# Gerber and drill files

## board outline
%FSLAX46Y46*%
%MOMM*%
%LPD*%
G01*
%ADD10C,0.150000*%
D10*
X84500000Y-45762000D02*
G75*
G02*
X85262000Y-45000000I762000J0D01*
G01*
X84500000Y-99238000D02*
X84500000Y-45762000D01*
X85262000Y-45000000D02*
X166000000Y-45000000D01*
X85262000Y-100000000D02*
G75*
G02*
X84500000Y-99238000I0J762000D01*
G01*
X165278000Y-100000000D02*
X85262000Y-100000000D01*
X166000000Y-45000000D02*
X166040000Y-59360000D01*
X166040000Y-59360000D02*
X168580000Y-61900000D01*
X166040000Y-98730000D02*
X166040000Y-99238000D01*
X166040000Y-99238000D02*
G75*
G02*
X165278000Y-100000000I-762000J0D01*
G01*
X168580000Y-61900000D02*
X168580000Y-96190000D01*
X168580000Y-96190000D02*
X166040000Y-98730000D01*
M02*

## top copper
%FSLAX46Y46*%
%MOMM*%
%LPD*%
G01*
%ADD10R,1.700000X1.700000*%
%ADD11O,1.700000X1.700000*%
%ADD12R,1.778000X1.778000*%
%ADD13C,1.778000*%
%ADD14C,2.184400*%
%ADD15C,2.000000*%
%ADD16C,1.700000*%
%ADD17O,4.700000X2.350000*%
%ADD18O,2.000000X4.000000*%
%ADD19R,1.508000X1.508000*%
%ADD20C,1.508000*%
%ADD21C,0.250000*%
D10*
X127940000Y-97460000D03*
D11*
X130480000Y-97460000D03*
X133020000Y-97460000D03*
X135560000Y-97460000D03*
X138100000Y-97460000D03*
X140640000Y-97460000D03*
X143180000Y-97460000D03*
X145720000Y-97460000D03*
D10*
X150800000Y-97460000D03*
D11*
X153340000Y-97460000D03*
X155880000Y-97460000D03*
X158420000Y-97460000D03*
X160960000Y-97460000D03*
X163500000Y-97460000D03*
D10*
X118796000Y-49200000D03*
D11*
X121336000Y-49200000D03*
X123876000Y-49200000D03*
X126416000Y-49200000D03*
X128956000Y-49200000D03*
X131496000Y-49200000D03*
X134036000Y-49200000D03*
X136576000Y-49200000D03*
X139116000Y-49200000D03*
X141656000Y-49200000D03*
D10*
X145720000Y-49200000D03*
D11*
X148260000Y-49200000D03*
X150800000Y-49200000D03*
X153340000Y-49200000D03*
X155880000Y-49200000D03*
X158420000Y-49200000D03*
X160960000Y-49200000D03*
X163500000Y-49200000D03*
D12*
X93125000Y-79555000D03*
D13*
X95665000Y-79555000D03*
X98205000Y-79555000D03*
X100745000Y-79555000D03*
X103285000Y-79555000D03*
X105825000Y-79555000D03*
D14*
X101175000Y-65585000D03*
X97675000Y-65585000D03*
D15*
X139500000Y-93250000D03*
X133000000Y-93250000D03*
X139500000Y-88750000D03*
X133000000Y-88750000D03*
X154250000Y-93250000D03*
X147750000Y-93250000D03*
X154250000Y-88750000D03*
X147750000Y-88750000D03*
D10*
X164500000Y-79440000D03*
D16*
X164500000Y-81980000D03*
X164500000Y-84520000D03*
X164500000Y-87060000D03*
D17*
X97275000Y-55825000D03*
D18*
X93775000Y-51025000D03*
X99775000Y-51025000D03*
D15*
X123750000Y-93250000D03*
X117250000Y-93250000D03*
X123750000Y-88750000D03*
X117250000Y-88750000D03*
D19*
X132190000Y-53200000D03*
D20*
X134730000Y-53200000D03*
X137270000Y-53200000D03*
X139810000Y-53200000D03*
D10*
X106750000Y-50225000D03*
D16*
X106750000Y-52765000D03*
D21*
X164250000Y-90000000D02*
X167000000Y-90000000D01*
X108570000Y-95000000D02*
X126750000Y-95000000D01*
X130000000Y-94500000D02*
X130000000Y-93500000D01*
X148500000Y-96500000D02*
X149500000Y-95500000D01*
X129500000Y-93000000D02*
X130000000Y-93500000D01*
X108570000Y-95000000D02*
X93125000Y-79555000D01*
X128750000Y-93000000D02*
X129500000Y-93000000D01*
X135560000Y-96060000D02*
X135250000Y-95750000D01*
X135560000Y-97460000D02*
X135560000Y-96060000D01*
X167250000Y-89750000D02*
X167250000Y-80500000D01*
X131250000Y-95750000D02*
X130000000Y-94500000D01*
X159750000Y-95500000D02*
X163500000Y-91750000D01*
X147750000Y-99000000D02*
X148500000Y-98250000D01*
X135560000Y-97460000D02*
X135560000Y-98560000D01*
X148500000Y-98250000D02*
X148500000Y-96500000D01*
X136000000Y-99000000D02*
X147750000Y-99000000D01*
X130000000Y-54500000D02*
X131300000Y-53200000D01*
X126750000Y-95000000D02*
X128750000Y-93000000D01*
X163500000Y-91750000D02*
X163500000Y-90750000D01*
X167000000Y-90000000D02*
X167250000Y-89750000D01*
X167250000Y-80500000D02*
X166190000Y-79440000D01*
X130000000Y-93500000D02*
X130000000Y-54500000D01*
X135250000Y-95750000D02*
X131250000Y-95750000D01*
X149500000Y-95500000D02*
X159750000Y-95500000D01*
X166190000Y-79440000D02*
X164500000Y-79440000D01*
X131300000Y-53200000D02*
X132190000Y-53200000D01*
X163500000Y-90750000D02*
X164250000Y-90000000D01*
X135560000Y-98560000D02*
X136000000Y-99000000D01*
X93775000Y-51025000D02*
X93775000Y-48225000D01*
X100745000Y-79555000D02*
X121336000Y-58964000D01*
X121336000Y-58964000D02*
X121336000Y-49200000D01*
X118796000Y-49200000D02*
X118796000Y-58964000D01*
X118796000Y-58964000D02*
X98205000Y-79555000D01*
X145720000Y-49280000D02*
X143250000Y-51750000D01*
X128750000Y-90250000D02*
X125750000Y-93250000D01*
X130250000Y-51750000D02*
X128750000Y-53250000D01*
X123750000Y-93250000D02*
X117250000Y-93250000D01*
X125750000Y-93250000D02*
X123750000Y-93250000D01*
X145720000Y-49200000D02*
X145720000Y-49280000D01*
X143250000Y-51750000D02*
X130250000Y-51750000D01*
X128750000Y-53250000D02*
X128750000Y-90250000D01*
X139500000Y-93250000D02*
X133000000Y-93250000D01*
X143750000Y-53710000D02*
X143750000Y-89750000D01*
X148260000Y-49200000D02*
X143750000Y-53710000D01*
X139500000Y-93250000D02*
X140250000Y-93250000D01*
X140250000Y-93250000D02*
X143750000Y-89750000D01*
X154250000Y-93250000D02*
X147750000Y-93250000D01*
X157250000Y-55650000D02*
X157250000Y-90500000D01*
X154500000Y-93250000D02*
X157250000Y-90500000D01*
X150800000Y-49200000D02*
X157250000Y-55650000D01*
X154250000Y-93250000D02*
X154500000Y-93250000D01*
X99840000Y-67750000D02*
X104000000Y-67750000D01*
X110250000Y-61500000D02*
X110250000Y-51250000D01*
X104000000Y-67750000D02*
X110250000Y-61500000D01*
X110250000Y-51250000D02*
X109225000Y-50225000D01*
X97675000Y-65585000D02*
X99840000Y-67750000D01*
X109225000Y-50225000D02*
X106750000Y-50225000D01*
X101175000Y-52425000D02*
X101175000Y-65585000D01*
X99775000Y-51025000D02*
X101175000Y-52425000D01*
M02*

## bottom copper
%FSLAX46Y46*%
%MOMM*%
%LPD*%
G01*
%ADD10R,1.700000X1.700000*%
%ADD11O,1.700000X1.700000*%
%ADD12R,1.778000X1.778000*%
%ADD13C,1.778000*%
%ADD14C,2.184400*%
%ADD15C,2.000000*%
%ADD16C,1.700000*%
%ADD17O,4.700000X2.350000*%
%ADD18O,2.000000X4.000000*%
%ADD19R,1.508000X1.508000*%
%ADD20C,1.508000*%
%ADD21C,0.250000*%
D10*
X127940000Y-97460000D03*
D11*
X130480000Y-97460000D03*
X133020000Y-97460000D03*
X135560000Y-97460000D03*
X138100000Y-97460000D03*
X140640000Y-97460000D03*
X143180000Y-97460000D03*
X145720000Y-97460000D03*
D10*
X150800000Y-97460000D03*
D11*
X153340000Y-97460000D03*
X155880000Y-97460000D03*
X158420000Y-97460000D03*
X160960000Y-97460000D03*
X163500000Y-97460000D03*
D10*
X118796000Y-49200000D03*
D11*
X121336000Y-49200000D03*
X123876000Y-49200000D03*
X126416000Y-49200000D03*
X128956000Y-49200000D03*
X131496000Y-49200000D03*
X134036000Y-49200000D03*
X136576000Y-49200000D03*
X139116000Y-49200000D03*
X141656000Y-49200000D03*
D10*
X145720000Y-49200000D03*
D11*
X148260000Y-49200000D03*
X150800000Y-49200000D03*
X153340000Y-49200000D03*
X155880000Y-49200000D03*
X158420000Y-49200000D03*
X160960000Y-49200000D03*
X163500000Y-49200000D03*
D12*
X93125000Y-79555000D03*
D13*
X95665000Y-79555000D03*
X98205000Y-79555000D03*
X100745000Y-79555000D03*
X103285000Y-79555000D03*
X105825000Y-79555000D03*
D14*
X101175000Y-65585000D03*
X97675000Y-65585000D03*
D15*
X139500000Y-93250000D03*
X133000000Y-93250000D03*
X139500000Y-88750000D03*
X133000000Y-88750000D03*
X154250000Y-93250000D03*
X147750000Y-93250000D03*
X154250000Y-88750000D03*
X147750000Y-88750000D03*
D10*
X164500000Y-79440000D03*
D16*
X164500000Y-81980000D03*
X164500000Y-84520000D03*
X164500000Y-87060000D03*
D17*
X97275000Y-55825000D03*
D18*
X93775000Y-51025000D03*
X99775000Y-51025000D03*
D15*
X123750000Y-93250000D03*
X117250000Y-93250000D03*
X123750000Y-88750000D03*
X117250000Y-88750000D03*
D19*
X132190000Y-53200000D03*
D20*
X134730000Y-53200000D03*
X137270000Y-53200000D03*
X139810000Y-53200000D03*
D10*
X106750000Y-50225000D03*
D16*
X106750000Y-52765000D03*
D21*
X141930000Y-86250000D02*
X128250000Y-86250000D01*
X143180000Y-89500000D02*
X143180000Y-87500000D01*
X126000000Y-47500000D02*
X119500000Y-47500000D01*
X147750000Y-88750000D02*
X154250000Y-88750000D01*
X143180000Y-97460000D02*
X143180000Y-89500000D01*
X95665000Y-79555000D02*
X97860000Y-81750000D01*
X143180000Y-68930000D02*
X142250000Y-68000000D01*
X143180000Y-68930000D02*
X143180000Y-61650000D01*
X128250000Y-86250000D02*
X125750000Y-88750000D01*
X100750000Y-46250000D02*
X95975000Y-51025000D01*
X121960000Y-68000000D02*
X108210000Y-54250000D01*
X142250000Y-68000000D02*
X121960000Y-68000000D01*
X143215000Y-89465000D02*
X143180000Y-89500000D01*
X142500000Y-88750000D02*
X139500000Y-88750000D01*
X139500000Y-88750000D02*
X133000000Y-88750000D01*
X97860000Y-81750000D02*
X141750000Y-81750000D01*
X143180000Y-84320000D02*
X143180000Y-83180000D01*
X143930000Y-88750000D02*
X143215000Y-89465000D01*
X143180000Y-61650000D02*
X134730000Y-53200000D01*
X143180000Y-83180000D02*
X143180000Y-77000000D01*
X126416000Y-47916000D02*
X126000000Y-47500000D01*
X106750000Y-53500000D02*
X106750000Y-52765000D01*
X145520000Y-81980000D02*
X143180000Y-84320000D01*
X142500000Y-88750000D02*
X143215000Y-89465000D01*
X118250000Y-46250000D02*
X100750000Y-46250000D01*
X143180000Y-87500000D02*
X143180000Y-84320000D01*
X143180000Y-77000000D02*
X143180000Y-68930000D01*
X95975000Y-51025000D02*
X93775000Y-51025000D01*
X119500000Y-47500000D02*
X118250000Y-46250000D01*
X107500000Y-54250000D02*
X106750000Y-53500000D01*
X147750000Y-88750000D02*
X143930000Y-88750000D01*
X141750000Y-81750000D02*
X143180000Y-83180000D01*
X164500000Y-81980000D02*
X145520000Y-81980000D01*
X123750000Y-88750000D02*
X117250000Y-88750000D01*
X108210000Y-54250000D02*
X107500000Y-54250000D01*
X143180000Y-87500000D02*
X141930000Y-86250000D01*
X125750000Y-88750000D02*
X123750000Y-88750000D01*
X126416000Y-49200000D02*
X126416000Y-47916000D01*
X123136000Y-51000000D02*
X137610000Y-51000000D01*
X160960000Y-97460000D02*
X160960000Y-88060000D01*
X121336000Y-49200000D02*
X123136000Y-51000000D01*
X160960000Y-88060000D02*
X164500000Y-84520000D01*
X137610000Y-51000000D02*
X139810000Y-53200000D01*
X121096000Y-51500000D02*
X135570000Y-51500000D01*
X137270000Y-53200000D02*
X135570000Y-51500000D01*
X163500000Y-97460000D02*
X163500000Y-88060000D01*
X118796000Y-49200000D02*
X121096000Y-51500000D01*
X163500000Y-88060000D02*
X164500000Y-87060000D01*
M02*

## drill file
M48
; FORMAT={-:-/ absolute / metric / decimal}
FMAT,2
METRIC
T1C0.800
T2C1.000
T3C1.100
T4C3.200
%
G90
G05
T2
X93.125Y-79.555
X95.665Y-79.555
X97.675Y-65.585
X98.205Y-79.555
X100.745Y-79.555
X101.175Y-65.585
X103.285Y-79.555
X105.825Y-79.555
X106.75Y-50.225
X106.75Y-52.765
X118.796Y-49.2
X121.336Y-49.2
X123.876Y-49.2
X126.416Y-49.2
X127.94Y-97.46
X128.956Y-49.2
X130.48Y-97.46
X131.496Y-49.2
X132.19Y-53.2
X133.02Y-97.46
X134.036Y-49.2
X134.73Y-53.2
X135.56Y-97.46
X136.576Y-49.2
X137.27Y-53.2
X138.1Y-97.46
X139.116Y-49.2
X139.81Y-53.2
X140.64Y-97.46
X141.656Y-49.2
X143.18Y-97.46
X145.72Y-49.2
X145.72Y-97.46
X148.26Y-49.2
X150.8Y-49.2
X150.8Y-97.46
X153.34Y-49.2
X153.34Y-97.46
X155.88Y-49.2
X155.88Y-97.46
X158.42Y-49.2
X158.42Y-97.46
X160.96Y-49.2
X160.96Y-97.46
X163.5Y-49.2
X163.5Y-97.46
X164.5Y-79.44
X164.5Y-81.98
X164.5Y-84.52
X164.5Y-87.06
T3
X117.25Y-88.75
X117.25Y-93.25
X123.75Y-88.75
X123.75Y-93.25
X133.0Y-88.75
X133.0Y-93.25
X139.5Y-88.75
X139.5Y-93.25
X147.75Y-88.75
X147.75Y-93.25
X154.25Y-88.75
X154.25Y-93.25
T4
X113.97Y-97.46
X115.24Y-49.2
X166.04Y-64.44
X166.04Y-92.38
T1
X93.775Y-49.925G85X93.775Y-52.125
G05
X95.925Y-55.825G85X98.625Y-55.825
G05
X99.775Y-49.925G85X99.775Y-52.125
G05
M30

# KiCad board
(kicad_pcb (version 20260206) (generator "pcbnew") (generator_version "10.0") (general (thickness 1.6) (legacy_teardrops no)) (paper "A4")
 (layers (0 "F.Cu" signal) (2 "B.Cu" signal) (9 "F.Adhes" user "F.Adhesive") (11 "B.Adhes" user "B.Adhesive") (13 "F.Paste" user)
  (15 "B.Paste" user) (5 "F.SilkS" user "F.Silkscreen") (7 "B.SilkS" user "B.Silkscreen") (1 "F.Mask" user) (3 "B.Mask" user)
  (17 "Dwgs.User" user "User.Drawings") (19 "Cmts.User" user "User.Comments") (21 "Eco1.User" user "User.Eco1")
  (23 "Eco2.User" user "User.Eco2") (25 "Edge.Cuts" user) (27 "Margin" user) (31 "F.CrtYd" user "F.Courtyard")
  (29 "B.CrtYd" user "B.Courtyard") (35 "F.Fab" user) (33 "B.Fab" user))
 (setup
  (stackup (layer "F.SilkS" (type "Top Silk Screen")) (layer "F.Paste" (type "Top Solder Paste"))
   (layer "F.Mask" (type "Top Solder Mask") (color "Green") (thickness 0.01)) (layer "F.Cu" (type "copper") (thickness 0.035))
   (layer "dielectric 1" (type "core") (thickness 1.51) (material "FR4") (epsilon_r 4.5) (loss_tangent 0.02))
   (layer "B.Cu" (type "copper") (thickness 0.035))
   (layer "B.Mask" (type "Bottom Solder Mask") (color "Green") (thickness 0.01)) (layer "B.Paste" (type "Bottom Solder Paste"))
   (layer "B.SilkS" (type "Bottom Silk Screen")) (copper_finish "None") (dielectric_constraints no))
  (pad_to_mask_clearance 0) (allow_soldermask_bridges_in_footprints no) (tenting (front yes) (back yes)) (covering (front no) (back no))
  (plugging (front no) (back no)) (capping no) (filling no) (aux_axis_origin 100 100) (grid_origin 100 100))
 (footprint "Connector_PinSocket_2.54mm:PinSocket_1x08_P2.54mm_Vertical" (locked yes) (layer "F.Cu") (at 127.94 97.46 90)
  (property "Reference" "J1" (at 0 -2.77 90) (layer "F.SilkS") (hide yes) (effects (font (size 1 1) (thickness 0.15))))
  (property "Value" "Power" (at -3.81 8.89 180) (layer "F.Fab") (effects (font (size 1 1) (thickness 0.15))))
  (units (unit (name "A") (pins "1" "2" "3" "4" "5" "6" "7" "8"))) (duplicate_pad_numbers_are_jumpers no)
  (pad "1" thru_hole rect (at 0 0 90) (size 1.7 1.7) (drill 1) (layers "*.Cu" "*.Mask") (remove_unused_layers no)
   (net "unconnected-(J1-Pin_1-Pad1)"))
  (pad "2" thru_hole oval (at 0 2.54 90) (size 1.7 1.7) (drill 1) (layers "*.Cu" "*.Mask") (remove_unused_layers no) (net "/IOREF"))
  (pad "3" thru_hole oval (at 0 5.08 90) (size 1.7 1.7) (drill 1) (layers "*.Cu" "*.Mask") (remove_unused_layers no) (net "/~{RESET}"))
  (pad "4" thru_hole oval (at 0 7.62 90) (size 1.7 1.7) (drill 1) (layers "*.Cu" "*.Mask") (remove_unused_layers no) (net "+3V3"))
  (pad "5" thru_hole oval (at 0 10.16 90) (size 1.7 1.7) (drill 1) (layers "*.Cu" "*.Mask") (remove_unused_layers no) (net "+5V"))
  (pad "6" thru_hole oval (at 0 12.7 90) (size 1.7 1.7) (drill 1) (layers "*.Cu" "*.Mask") (remove_unused_layers no) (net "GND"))
  (pad "7" thru_hole oval (at 0 15.24 90) (size 1.7 1.7) (drill 1) (layers "*.Cu" "*.Mask") (remove_unused_layers no) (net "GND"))
  (pad "8" thru_hole oval (at 0 17.78 90) (size 1.7 1.7) (drill 1) (layers "*.Cu" "*.Mask") (remove_unused_layers no) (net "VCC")))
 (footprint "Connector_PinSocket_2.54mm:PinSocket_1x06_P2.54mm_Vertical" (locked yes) (layer "F.Cu") (at 150.8 97.46 90)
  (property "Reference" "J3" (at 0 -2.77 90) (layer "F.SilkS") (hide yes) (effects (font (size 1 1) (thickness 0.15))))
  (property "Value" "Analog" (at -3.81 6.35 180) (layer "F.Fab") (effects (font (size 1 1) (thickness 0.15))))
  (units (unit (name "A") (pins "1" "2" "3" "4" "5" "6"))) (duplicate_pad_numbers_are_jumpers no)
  (pad "1" thru_hole rect (at 0 0 90) (size 1.7 1.7) (drill 1) (layers "*.Cu" "*.Mask") (remove_unused_layers no) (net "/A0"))
  (pad "2" thru_hole oval (at 0 2.54 90) (size 1.7 1.7) (drill 1) (layers "*.Cu" "*.Mask") (remove_unused_layers no) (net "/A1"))
  (pad "3" thru_hole oval (at 0 5.08 90) (size 1.7 1.7) (drill 1) (layers "*.Cu" "*.Mask") (remove_unused_layers no) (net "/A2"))
  (pad "4" thru_hole oval (at 0 7.62 90) (size 1.7 1.7) (drill 1) (layers "*.Cu" "*.Mask") (remove_unused_layers no) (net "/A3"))
  (pad "5" thru_hole oval (at 0 10.16 90) (size 1.7 1.7) (drill 1) (layers "*.Cu" "*.Mask") (remove_unused_layers no) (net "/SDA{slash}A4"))
  (pad "6" thru_hole oval (at 0 12.7 90) (size 1.7 1.7) (drill 1) (layers "*.Cu" "*.Mask") (remove_unused_layers no) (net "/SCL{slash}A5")))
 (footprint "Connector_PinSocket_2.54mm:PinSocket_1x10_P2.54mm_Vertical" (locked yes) (layer "F.Cu") (at 118.796 49.2 90)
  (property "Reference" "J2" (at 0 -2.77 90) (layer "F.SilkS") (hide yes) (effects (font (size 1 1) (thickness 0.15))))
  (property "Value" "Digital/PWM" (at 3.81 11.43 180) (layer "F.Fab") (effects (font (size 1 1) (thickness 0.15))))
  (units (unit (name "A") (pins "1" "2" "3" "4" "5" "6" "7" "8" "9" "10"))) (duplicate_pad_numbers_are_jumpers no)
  (pad "1" thru_hole rect (at 0 0 90) (size 1.7 1.7) (drill 1) (layers "*.Cu" "*.Mask") (remove_unused_layers no) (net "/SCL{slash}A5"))
  (pad "2" thru_hole oval (at 0 2.54 90) (size 1.7 1.7) (drill 1) (layers "*.Cu" "*.Mask") (remove_unused_layers no) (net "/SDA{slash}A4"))
  (pad "3" thru_hole oval (at 0 5.08 90) (size 1.7 1.7) (drill 1) (layers "*.Cu" "*.Mask") (remove_unused_layers no) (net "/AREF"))
  (pad "4" thru_hole oval (at 0 7.62 90) (size 1.7 1.7) (drill 1) (layers "*.Cu" "*.Mask") (remove_unused_layers no) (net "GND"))
  (pad "5" thru_hole oval (at 0 10.16 90) (size 1.7 1.7) (drill 1) (layers "*.Cu" "*.Mask") (remove_unused_layers no) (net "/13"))
  (pad "6" thru_hole oval (at 0 12.7 90) (size 1.7 1.7) (drill 1) (layers "*.Cu" "*.Mask") (remove_unused_layers no) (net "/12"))
  (pad "7" thru_hole oval (at 0 15.24 90) (size 1.7 1.7) (drill 1) (layers "*.Cu" "*.Mask") (remove_unused_layers no) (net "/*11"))
  (pad "8" thru_hole oval (at 0 17.78 90) (size 1.7 1.7) (drill 1) (layers "*.Cu" "*.Mask") (remove_unused_layers no) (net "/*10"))
  (pad "9" thru_hole oval (at 0 20.32 90) (size 1.7 1.7) (drill 1) (layers "*.Cu" "*.Mask") (remove_unused_layers no) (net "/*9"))
  (pad "10" thru_hole oval (at 0 22.86 90) (size 1.7 1.7) (drill 1) (layers "*.Cu" "*.Mask") (remove_unused_layers no) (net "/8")))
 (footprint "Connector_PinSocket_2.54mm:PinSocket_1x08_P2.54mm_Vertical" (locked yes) (layer "F.Cu") (at 145.72 49.2 90)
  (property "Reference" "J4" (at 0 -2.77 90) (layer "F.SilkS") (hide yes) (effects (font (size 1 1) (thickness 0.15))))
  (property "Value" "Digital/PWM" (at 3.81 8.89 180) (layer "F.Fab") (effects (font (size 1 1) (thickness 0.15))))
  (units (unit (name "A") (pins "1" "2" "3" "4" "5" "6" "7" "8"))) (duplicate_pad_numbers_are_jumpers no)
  (pad "1" thru_hole rect (at 0 0 90) (size 1.7 1.7) (drill 1) (layers "*.Cu" "*.Mask") (remove_unused_layers no) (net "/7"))
  (pad "2" thru_hole oval (at 0 2.54 90) (size 1.7 1.7) (drill 1) (layers "*.Cu" "*.Mask") (remove_unused_layers no) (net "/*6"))
  (pad "3" thru_hole oval (at 0 5.08 90) (size 1.7 1.7) (drill 1) (layers "*.Cu" "*.Mask") (remove_unused_layers no) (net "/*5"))
  (pad "4" thru_hole oval (at 0 7.62 90) (size 1.7 1.7) (drill 1) (layers "*.Cu" "*.Mask") (remove_unused_layers no) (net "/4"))
  (pad "5" thru_hole oval (at 0 10.16 90) (size 1.7 1.7) (drill 1) (layers "*.Cu" "*.Mask") (remove_unused_layers no) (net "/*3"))
  (pad "6" thru_hole oval (at 0 12.7 90) (size 1.7 1.7) (drill 1) (layers "*.Cu" "*.Mask") (remove_unused_layers no) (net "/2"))
  (pad "7" thru_hole oval (at 0 15.24 90) (size 1.7 1.7) (drill 1) (layers "*.Cu" "*.Mask") (remove_unused_layers no) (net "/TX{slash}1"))
  (pad "8" thru_hole oval (at 0 17.78 90) (size 1.7 1.7) (drill 1) (layers "*.Cu" "*.Mask") (remove_unused_layers no) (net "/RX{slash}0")))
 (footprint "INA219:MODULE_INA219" (layer "F.Cu") (at 99.475 71.935)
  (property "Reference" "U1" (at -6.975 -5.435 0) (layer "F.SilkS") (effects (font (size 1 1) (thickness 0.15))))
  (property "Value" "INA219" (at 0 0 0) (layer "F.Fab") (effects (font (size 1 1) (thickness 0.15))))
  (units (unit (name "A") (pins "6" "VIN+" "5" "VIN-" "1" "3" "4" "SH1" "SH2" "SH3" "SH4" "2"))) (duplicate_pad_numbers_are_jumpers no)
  (pad "1" thru_hole rect (at -6.35 7.62) (size 1.778 1.778) (drill 1) (layers "*.Cu" "*.Mask") (remove_unused_layers no) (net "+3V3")
   (solder_mask_margin 0.102))
  (pad "2" thru_hole circle (at -3.81 7.62) (size 1.778 1.778) (drill 1) (layers "*.Cu" "*.Mask") (remove_unused_layers no) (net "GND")
   (solder_mask_margin 0.102))
  (pad "3" thru_hole circle (at -1.27 7.62) (size 1.778 1.778) (drill 1) (layers "*.Cu" "*.Mask") (remove_unused_layers no)
   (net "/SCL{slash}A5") (solder_mask_margin 0.102))
  (pad "4" thru_hole circle (at 1.27 7.62) (size 1.778 1.778) (drill 1) (layers "*.Cu" "*.Mask") (remove_unused_layers no)
   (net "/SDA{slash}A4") (solder_mask_margin 0.102))
  (pad "5" thru_hole circle (at 3.81 7.62) (size 1.778 1.778) (drill 1) (layers "*.Cu" "*.Mask") (remove_unused_layers no)
   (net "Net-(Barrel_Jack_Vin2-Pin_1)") (solder_mask_margin 0.102))
  (pad "6" thru_hole circle (at 6.35 7.62) (size 1.778 1.778) (drill 1) (layers "*.Cu" "*.Mask") (remove_unused_layers no)
   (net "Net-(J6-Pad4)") (solder_mask_margin 0.102))
  (pad "VIN+" thru_hole circle (at 1.7 -6.35) (size 2.1844 2.1844) (drill 1) (layers "*.Cu" "*.Mask") (remove_unused_layers no)
   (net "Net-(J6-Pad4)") (solder_mask_margin 0.102))
  (pad "VIN-" thru_hole circle (at -1.8 -6.35) (size 2.1844 2.1844) (drill 1) (layers "*.Cu" "*.Mask") (remove_unused_layers no)
   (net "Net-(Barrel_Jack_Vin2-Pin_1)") (solder_mask_margin 0.102)))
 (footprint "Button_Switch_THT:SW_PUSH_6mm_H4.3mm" (layer "F.Cu") (at 139.5 93.25 180)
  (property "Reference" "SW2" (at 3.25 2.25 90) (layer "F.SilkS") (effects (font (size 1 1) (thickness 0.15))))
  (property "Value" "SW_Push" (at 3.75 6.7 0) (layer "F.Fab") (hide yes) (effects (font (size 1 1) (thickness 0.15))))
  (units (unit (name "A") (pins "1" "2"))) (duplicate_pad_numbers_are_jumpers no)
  (pad "1" thru_hole circle (at 0 0 270) (size 2 2) (drill 1.1) (layers "*.Cu" "*.Mask") (remove_unused_layers no) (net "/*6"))
  (pad "1" thru_hole circle (at 6.5 0 270) (size 2 2) (drill 1.1) (layers "*.Cu" "*.Mask") (remove_unused_layers no) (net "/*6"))
  (pad "2" thru_hole circle (at 0 4.5 270) (size 2 2) (drill 1.1) (layers "*.Cu" "*.Mask") (remove_unused_layers no) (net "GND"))
  (pad "2" thru_hole circle (at 6.5 4.5 270) (size 2 2) (drill 1.1) (layers "*.Cu" "*.Mask") (remove_unused_layers no) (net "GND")))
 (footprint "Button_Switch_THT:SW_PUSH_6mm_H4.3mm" (layer "F.Cu") (at 154.25 93.25 180)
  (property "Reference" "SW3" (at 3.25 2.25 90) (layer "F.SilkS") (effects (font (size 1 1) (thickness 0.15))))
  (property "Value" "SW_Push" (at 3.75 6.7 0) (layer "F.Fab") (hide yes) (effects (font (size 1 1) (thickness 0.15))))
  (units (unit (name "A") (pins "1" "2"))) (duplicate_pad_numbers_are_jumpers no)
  (pad "1" thru_hole circle (at 0 0 270) (size 2 2) (drill 1.1) (layers "*.Cu" "*.Mask") (remove_unused_layers no) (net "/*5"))
  (pad "1" thru_hole circle (at 6.5 0 270) (size 2 2) (drill 1.1) (layers "*.Cu" "*.Mask") (remove_unused_layers no) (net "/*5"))
  (pad "2" thru_hole circle (at 0 4.5 270) (size 2 2) (drill 1.1) (layers "*.Cu" "*.Mask") (remove_unused_layers no) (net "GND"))
  (pad "2" thru_hole circle (at 6.5 4.5 270) (size 2 2) (drill 1.1) (layers "*.Cu" "*.Mask") (remove_unused_layers no) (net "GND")))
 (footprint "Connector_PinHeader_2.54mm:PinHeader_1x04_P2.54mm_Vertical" (layer "F.Cu") (at 164.5 79.44)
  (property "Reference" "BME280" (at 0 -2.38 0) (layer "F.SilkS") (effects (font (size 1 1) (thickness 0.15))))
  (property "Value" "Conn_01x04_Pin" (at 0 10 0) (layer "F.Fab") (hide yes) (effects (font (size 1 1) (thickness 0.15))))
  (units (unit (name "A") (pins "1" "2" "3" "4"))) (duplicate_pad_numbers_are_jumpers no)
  (pad "1" thru_hole rect (at 0 0) (size 1.7 1.7) (drill 1) (layers "*.Cu" "*.Mask") (remove_unused_layers no) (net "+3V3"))
  (pad "2" thru_hole circle (at 0 2.54) (size 1.7 1.7) (drill 1) (layers "*.Cu" "*.Mask") (remove_unused_layers no) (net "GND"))
  (pad "3" thru_hole circle (at 0 5.08) (size 1.7 1.7) (drill 1) (layers "*.Cu" "*.Mask") (remove_unused_layers no) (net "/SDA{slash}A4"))
  (pad "4" thru_hole circle (at 0 7.62) (size 1.7 1.7) (drill 1) (layers "*.Cu" "*.Mask") (remove_unused_layers no) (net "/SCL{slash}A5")))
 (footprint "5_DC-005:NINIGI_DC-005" (layer "F.Cu") (at 97.275 51.025)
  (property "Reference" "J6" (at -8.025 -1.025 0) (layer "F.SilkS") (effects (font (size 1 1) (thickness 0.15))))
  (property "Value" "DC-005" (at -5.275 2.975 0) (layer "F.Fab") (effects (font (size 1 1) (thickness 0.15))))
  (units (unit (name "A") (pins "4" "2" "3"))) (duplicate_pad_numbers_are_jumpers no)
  (pad "2" thru_hole oval (at 0 4.8) (size 4.7 2.35) (drill oval 3.5 0.8) (layers "*.Cu" "*.Mask") (remove_unused_layers no)
   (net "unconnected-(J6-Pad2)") (solder_mask_margin 0.102))
  (pad "3" thru_hole oval (at -3.5 0) (size 2 4) (drill oval 0.8 3) (layers "*.Cu" "*.Mask") (remove_unused_layers no) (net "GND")
   (solder_mask_margin 0.102))
  (pad "4" thru_hole oval (at 2.5 0) (size 2 4) (drill oval 0.8 3) (layers "*.Cu" "*.Mask") (remove_unused_layers no) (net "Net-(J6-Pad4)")
   (solder_mask_margin 0.102)))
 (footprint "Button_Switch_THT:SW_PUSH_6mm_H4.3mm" (layer "F.Cu") (at 123.75 93.25 180)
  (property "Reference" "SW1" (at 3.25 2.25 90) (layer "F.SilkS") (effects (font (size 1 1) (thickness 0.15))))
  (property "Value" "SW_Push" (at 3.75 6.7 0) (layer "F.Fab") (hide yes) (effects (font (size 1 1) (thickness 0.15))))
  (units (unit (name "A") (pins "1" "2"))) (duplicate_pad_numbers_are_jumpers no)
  (pad "1" thru_hole circle (at 0 0 270) (size 2 2) (drill 1.1) (layers "*.Cu" "*.Mask") (remove_unused_layers no) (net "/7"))
  (pad "1" thru_hole circle (at 6.5 0 270) (size 2 2) (drill 1.1) (layers "*.Cu" "*.Mask") (remove_unused_layers no) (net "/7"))
  (pad "2" thru_hole circle (at 0 4.5 270) (size 2 2) (drill 1.1) (layers "*.Cu" "*.Mask") (remove_unused_layers no) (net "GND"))
  (pad "2" thru_hole circle (at 6.5 4.5 270) (size 2 2) (drill 1.1) (layers "*.Cu" "*.Mask") (remove_unused_layers no) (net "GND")))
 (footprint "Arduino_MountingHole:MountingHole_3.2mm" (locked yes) (layer "F.Cu") (at 115.24 49.2)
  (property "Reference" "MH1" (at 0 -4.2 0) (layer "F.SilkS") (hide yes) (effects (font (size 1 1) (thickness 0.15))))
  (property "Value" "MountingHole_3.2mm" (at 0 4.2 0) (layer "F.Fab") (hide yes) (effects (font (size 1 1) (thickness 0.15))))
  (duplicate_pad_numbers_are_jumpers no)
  (pad "" np_thru_hole circle (at 0 0) (size 3.2 3.2) (drill 3.2) (layers "*.Cu" "*.Mask")))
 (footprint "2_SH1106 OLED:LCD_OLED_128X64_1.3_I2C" (layer "F.Cu") (at 136 68.75)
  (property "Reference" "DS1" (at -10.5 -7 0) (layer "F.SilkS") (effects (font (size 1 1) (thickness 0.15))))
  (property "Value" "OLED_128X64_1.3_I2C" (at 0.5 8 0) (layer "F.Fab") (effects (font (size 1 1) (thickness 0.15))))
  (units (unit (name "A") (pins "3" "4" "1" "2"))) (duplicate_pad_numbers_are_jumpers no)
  (pad "1" thru_hole rect (at -3.81 -15.55) (size 1.508 1.508) (drill 1) (layers "*.Cu" "*.Mask") (remove_unused_layers no) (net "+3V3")
   (solder_mask_margin 0.102))
  (pad "2" thru_hole circle (at -1.27 -15.55) (size 1.508 1.508) (drill 1) (layers "*.Cu" "*.Mask") (remove_unused_layers no) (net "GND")
   (solder_mask_margin 0.102))
  (pad "3" thru_hole circle (at 1.27 -15.55) (size 1.508 1.508) (drill 1) (layers "*.Cu" "*.Mask") (remove_unused_layers no)
   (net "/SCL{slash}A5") (solder_mask_margin 0.102))
  (pad "4" thru_hole circle (at 3.81 -15.55) (size 1.508 1.508) (drill 1) (layers "*.Cu" "*.Mask") (remove_unused_layers no)
   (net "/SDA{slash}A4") (solder_mask_margin 0.102)))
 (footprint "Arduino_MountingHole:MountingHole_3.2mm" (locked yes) (layer "F.Cu") (at 113.97 97.46)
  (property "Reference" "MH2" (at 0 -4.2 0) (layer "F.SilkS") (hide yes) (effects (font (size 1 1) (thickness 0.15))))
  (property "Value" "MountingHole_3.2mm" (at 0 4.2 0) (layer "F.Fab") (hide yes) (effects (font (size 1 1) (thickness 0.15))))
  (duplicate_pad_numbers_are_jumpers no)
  (pad "" np_thru_hole circle (at 0 0) (size 3.2 3.2) (drill 3.2) (layers "*.Cu" "*.Mask")))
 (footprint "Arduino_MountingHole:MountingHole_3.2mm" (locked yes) (layer "F.Cu") (at 166.04 64.44)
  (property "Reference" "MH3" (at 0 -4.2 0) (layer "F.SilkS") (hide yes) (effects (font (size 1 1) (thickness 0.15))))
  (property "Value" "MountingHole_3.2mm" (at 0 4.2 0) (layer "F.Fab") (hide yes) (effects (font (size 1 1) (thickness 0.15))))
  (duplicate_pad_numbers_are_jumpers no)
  (pad "" np_thru_hole circle (at 0 0) (size 3.2 3.2) (drill 3.2) (layers "*.Cu" "*.Mask")))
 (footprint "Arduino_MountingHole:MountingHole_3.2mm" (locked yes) (layer "F.Cu") (at 166.04 92.38)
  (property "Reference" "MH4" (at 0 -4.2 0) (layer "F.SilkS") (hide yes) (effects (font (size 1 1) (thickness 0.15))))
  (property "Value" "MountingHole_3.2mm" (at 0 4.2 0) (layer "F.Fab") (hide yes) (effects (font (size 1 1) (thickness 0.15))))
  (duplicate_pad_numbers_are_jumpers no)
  (pad "" np_thru_hole circle (at 0 0) (size 3.2 3.2) (drill 3.2) (layers "*.Cu" "*.Mask")))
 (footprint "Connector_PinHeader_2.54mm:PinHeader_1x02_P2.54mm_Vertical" (layer "F.Cu") (at 106.75 50.225)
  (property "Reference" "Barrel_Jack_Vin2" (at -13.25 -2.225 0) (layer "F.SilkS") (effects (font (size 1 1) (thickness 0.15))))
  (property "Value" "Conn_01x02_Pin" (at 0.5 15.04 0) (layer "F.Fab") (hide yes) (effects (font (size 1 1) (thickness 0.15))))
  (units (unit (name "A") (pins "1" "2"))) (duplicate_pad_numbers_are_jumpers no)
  (pad "1" thru_hole rect (at 0 0) (size 1.7 1.7) (drill 1) (layers "*.Cu" "*.Mask") (remove_unused_layers no)
   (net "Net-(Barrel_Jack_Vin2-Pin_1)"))
  (pad "2" thru_hole circle (at 0 2.54) (size 1.7 1.7) (drill 1) (layers "*.Cu" "*.Mask") (remove_unused_layers no) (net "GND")))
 (gr_arc (start 84.5 45.762) (mid 84.723185 45.223185) (end 85.262 45) (stroke (width 0.15) (type solid)) (locked yes) (layer "Edge.Cuts"))
 (gr_line (start 84.5 99.238) (end 84.5 45.762) (stroke (width 0.15) (type solid)) (locked yes) (layer "Edge.Cuts"))
 (gr_line (start 85.262 45) (end 166 45) (stroke (width 0.15) (type solid)) (locked yes) (layer "Edge.Cuts"))
 (gr_arc (start 85.262 100) (mid 84.723185 99.776815) (end 84.5 99.238) (stroke (width 0.15) (type solid)) (locked yes) (layer "Edge.Cuts"))
 (gr_line (start 165.278 100) (end 85.262 100) (stroke (width 0.15) (type solid)) (locked yes) (layer "Edge.Cuts"))
 (gr_line (start 166 45) (end 166.04 59.36) (stroke (width 0.15) (type solid)) (locked yes) (layer "Edge.Cuts"))
 (gr_line (start 166.04 59.36) (end 168.58 61.9) (stroke (width 0.15) (type solid)) (locked yes) (layer "Edge.Cuts"))
 (gr_line (start 166.04 98.73) (end 166.04 99.238) (stroke (width 0.15) (type solid)) (locked yes) (layer "Edge.Cuts"))
 (gr_arc (start 166.04 99.238) (mid 165.816815 99.776815) (end 165.278 100) (stroke (width 0.15) (type solid)) (locked yes)
  (layer "Edge.Cuts"))
 (gr_line (start 168.58 61.9) (end 168.58 96.19) (stroke (width 0.15) (type solid)) (locked yes) (layer "Edge.Cuts"))
 (gr_line (start 168.58 96.19) (end 166.04 98.73) (stroke (width 0.15) (type solid)) (locked yes) (layer "Edge.Cuts"))
 (segment (start 164.25 90) (end 167 90) (width 0.25) (layer "F.Cu") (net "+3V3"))
 (segment (start 108.57 95) (end 126.75 95) (width 0.25) (layer "F.Cu") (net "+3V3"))
 (segment (start 130 94.5) (end 130 93.5) (width 0.25) (layer "F.Cu") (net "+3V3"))
 (segment (start 148.5 96.5) (end 149.5 95.5) (width 0.25) (layer "F.Cu") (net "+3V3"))
 (segment (start 129.5 93) (end 130 93.5) (width 0.25) (layer "F.Cu") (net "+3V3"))
 (segment (start 108.57 95) (end 93.125 79.555) (width 0.25) (layer "F.Cu") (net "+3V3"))
 (segment (start 128.75 93) (end 129.5 93) (width 0.25) (layer "F.Cu") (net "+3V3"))
 (segment (start 135.56 96.06) (end 135.25 95.75) (width 0.25) (layer "F.Cu") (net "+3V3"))
 (segment (start 135.56 97.46) (end 135.56 96.06) (width 0.25) (layer "F.Cu") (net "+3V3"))
 (segment (start 167.25 89.75) (end 167.25 80.5) (width 0.25) (layer "F.Cu") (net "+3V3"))
 (segment (start 131.25 95.75) (end 130 94.5) (width 0.25) (layer "F.Cu") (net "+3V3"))
 (segment (start 159.75 95.5) (end 163.5 91.75) (width 0.25) (layer "F.Cu") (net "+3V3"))
 (segment (start 147.75 99) (end 148.5 98.25) (width 0.25) (layer "F.Cu") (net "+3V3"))
 (segment (start 135.56 97.46) (end 135.56 98.56) (width 0.25) (layer "F.Cu") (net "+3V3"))
 (segment (start 148.5 98.25) (end 148.5 96.5) (width 0.25) (layer "F.Cu") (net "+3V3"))
 (segment (start 136 99) (end 147.75 99) (width 0.25) (layer "F.Cu") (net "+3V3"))
 (segment (start 130 54.5) (end 131.3 53.2) (width 0.25) (layer "F.Cu") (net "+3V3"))
 (segment (start 126.75 95) (end 128.75 93) (width 0.25) (layer "F.Cu") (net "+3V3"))
 (segment (start 163.5 91.75) (end 163.5 90.75) (width 0.25) (layer "F.Cu") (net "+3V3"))
 (segment (start 167 90) (end 167.25 89.75) (width 0.25) (layer "F.Cu") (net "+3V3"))
 (segment (start 167.25 80.5) (end 166.19 79.44) (width 0.25) (layer "F.Cu") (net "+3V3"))
 (segment (start 130 93.5) (end 130 54.5) (width 0.25) (layer "F.Cu") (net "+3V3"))
 (segment (start 135.25 95.75) (end 131.25 95.75) (width 0.25) (layer "F.Cu") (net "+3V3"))
 (segment (start 149.5 95.5) (end 159.75 95.5) (width 0.25) (layer "F.Cu") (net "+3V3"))
 (segment (start 166.19 79.44) (end 164.5 79.44) (width 0.25) (layer "F.Cu") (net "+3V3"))
 (segment (start 131.3 53.2) (end 132.19 53.2) (width 0.25) (layer "F.Cu") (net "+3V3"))
 (segment (start 163.5 90.75) (end 164.25 90) (width 0.25) (layer "F.Cu") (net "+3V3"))
 (segment (start 135.56 98.56) (end 136 99) (width 0.25) (layer "F.Cu") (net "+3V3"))
 (segment (start 93.775 51.025) (end 93.775 48.225) (width 0.25) (layer "F.Cu") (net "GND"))
 (segment (start 141.93 86.25) (end 128.25 86.25) (width 0.25) (layer "B.Cu") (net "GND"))
 (segment (start 143.18 89.5) (end 143.18 87.5) (width 0.25) (layer "B.Cu") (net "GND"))
 (segment (start 126 47.5) (end 119.5 47.5) (width 0.25) (layer "B.Cu") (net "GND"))
 (segment (start 147.75 88.75) (end 154.25 88.75) (width 0.25) (layer "B.Cu") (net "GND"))
 (segment (start 143.18 97.46) (end 143.18 89.5) (width 0.25) (layer "B.Cu") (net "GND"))
 (segment (start 95.665 79.555) (end 97.86 81.75) (width 0.25) (layer "B.Cu") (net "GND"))
 (segment (start 143.18 68.93) (end 142.25 68) (width 0.25) (layer "B.Cu") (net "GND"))
 (segment (start 143.18 68.93) (end 143.18 61.65) (width 0.25) (layer "B.Cu") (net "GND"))
 (segment (start 128.25 86.25) (end 125.75 88.75) (width 0.25) (layer "B.Cu") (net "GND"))
 (segment (start 100.75 46.25) (end 95.975 51.025) (width 0.25) (layer "B.Cu") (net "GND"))
 (segment (start 121.96 68) (end 108.21 54.25) (width 0.25) (layer "B.Cu") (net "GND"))
 (segment (start 142.25 68) (end 121.96 68) (width 0.25) (layer "B.Cu") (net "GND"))
 (segment (start 143.215 89.465) (end 143.18 89.5) (width 0.25) (layer "B.Cu") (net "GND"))
 (segment (start 142.5 88.75) (end 139.5 88.75) (width 0.25) (layer "B.Cu") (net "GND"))
 (segment (start 139.5 88.75) (end 133 88.75) (width 0.25) (layer "B.Cu") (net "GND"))
 (segment (start 97.86 81.75) (end 141.75 81.75) (width 0.25) (layer "B.Cu") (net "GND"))
 (segment (start 143.18 84.32) (end 143.18 83.18) (width 0.25) (layer "B.Cu") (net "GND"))
 (segment (start 143.93 88.75) (end 143.215 89.465) (width 0.25) (layer "B.Cu") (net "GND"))
 (segment (start 143.18 61.65) (end 134.73 53.2) (width 0.25) (layer "B.Cu") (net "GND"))
 (segment (start 143.18 83.18) (end 143.18 77) (width 0.25) (layer "B.Cu") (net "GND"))
 (segment (start 126.416 47.916) (end 126 47.5) (width 0.25) (layer "B.Cu") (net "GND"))
 (segment (start 106.75 53.5) (end 106.75 52.765) (width 0.25) (layer "B.Cu") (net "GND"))
 (segment (start 145.52 81.98) (end 143.18 84.32) (width 0.25) (layer "B.Cu") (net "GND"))
 (segment (start 142.5 88.75) (end 143.215 89.465) (width 0.25) (layer "B.Cu") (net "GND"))
 (segment (start 118.25 46.25) (end 100.75 46.25) (width 0.25) (layer "B.Cu") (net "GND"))
 (segment (start 143.18 87.5) (end 143.18 84.32) (width 0.25) (layer "B.Cu") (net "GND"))
 (segment (start 143.18 77) (end 143.18 68.93) (width 0.25) (layer "B.Cu") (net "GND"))
 (segment (start 95.975 51.025) (end 93.775 51.025) (width 0.25) (layer "B.Cu") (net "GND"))
 (segment (start 119.5 47.5) (end 118.25 46.25) (width 0.25) (layer "B.Cu") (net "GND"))
 (segment (start 107.5 54.25) (end 106.75 53.5) (width 0.25) (layer "B.Cu") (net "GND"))
 (segment (start 147.75 88.75) (end 143.93 88.75) (width 0.25) (layer "B.Cu") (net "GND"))
 (segment (start 141.75 81.75) (end 143.18 83.18) (width 0.25) (layer "B.Cu") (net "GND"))
 (segment (start 164.5 81.98) (end 145.52 81.98) (width 0.25) (layer "B.Cu") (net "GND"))
 (segment (start 123.75 88.75) (end 117.25 88.75) (width 0.25) (layer "B.Cu") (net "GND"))
 (segment (start 108.21 54.25) (end 107.5 54.25) (width 0.25) (layer "B.Cu") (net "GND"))
 (segment (start 143.18 87.5) (end 141.93 86.25) (width 0.25) (layer "B.Cu") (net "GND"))
 (segment (start 125.75 88.75) (end 123.75 88.75) (width 0.25) (layer "B.Cu") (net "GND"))
 (segment (start 126.416 49.2) (end 126.416 47.916) (width 0.25) (layer "B.Cu") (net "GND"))
 (segment (start 100.745 79.555) (end 121.336 58.964) (width 0.25) (layer "F.Cu") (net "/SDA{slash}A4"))
 (segment (start 121.336 58.964) (end 121.336 49.2) (width 0.25) (layer "F.Cu") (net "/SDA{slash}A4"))
 (segment (start 123.136 51) (end 137.61 51) (width 0.25) (layer "B.Cu") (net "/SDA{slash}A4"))
 (segment (start 160.96 97.46) (end 160.96 88.06) (width 0.25) (layer "B.Cu") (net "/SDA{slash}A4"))
 (segment (start 121.336 49.2) (end 123.136 51) (width 0.25) (layer "B.Cu") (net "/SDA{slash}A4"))
 (segment (start 160.96 88.06) (end 164.5 84.52) (width 0.25) (layer "B.Cu") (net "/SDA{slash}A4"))
 (segment (start 137.61 51) (end 139.81 53.2) (width 0.25) (layer "B.Cu") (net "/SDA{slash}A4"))
 (segment (start 118.796 49.2) (end 118.796 58.964) (width 0.25) (layer "F.Cu") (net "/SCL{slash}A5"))
 (segment (start 118.796 58.964) (end 98.205 79.555) (width 0.25) (layer "F.Cu") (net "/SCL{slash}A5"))
 (segment (start 121.096 51.5) (end 135.57 51.5) (width 0.25) (layer "B.Cu") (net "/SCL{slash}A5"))
 (segment (start 137.27 53.2) (end 135.57 51.5) (width 0.25) (layer "B.Cu") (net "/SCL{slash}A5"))
 (segment (start 163.5 97.46) (end 163.5 88.06) (width 0.25) (layer "B.Cu") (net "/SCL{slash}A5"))
 (segment (start 118.796 49.2) (end 121.096 51.5) (width 0.25) (layer "B.Cu") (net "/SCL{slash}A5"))
 (segment (start 163.5 88.06) (end 164.5 87.06) (width 0.25) (layer "B.Cu") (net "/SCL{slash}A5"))
 (segment (start 145.72 49.28) (end 143.25 51.75) (width 0.25) (layer "F.Cu") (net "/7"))
 (segment (start 128.75 90.25) (end 125.75 93.25) (width 0.25) (layer "F.Cu") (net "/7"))
 (segment (start 130.25 51.75) (end 128.75 53.25) (width 0.25) (layer "F.Cu") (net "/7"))
 (segment (start 123.75 93.25) (end 117.25 93.25) (width 0.25) (layer "F.Cu") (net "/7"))
 (segment (start 125.75 93.25) (end 123.75 93.25) (width 0.25) (layer "F.Cu") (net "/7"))
 (segment (start 145.72 49.2) (end 145.72 49.28) (width 0.25) (layer "F.Cu") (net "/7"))
 (segment (start 143.25 51.75) (end 130.25 51.75) (width 0.25) (layer "F.Cu") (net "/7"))
 (segment (start 128.75 53.25) (end 128.75 90.25) (width 0.25) (layer "F.Cu") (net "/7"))
 (segment (start 139.5 93.25) (end 133 93.25) (width 0.25) (layer "F.Cu") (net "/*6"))
 (segment (start 143.75 53.71) (end 143.75 89.75) (width 0.25) (layer "F.Cu") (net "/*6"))
 (segment (start 148.26 49.2) (end 143.75 53.71) (width 0.25) (layer "F.Cu") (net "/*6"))
 (segment (start 139.5 93.25) (end 140.25 93.25) (width 0.25) (layer "F.Cu") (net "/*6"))
 (segment (start 140.25 93.25) (end 143.75 89.75) (width 0.25) (layer "F.Cu") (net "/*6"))
 (segment (start 154.25 93.25) (end 147.75 93.25) (width 0.25) (layer "F.Cu") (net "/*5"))
 (segment (start 157.25 55.65) (end 157.25 90.5) (width 0.25) (layer "F.Cu") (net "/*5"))
 (segment (start 154.5 93.25) (end 157.25 90.5) (width 0.25) (layer "F.Cu") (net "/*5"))
 (segment (start 150.8 49.2) (end 157.25 55.65) (width 0.25) (layer "F.Cu") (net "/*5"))
 (segment (start 154.25 93.25) (end 154.5 93.25) (width 0.25) (layer "F.Cu") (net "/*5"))
 (segment (start 99.84 67.75) (end 104 67.75) (width 0.25) (layer "F.Cu") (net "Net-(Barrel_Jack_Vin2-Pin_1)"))
 (segment (start 110.25 61.5) (end 110.25 51.25) (width 0.25) (layer "F.Cu") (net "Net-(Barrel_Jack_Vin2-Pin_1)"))
 (segment (start 104 67.75) (end 110.25 61.5) (width 0.25) (layer "F.Cu") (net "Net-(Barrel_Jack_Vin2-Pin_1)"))
 (segment (start 110.25 51.25) (end 109.225 50.225) (width 0.25) (layer "F.Cu") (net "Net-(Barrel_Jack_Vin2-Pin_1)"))
 (segment (start 97.675 65.585) (end 99.84 67.75) (width 0.25) (layer "F.Cu") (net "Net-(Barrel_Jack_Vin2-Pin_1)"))
 (segment (start 109.225 50.225) (end 106.75 50.225) (width 0.25) (layer "F.Cu") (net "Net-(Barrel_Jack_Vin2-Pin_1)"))
 (segment (start 101.175 52.425) (end 101.175 65.585) (width 0.25) (layer "F.Cu") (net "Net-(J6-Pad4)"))
 (segment (start 99.775 51.025) (end 101.175 52.425) (width 0.25) (layer "F.Cu") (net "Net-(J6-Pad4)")))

